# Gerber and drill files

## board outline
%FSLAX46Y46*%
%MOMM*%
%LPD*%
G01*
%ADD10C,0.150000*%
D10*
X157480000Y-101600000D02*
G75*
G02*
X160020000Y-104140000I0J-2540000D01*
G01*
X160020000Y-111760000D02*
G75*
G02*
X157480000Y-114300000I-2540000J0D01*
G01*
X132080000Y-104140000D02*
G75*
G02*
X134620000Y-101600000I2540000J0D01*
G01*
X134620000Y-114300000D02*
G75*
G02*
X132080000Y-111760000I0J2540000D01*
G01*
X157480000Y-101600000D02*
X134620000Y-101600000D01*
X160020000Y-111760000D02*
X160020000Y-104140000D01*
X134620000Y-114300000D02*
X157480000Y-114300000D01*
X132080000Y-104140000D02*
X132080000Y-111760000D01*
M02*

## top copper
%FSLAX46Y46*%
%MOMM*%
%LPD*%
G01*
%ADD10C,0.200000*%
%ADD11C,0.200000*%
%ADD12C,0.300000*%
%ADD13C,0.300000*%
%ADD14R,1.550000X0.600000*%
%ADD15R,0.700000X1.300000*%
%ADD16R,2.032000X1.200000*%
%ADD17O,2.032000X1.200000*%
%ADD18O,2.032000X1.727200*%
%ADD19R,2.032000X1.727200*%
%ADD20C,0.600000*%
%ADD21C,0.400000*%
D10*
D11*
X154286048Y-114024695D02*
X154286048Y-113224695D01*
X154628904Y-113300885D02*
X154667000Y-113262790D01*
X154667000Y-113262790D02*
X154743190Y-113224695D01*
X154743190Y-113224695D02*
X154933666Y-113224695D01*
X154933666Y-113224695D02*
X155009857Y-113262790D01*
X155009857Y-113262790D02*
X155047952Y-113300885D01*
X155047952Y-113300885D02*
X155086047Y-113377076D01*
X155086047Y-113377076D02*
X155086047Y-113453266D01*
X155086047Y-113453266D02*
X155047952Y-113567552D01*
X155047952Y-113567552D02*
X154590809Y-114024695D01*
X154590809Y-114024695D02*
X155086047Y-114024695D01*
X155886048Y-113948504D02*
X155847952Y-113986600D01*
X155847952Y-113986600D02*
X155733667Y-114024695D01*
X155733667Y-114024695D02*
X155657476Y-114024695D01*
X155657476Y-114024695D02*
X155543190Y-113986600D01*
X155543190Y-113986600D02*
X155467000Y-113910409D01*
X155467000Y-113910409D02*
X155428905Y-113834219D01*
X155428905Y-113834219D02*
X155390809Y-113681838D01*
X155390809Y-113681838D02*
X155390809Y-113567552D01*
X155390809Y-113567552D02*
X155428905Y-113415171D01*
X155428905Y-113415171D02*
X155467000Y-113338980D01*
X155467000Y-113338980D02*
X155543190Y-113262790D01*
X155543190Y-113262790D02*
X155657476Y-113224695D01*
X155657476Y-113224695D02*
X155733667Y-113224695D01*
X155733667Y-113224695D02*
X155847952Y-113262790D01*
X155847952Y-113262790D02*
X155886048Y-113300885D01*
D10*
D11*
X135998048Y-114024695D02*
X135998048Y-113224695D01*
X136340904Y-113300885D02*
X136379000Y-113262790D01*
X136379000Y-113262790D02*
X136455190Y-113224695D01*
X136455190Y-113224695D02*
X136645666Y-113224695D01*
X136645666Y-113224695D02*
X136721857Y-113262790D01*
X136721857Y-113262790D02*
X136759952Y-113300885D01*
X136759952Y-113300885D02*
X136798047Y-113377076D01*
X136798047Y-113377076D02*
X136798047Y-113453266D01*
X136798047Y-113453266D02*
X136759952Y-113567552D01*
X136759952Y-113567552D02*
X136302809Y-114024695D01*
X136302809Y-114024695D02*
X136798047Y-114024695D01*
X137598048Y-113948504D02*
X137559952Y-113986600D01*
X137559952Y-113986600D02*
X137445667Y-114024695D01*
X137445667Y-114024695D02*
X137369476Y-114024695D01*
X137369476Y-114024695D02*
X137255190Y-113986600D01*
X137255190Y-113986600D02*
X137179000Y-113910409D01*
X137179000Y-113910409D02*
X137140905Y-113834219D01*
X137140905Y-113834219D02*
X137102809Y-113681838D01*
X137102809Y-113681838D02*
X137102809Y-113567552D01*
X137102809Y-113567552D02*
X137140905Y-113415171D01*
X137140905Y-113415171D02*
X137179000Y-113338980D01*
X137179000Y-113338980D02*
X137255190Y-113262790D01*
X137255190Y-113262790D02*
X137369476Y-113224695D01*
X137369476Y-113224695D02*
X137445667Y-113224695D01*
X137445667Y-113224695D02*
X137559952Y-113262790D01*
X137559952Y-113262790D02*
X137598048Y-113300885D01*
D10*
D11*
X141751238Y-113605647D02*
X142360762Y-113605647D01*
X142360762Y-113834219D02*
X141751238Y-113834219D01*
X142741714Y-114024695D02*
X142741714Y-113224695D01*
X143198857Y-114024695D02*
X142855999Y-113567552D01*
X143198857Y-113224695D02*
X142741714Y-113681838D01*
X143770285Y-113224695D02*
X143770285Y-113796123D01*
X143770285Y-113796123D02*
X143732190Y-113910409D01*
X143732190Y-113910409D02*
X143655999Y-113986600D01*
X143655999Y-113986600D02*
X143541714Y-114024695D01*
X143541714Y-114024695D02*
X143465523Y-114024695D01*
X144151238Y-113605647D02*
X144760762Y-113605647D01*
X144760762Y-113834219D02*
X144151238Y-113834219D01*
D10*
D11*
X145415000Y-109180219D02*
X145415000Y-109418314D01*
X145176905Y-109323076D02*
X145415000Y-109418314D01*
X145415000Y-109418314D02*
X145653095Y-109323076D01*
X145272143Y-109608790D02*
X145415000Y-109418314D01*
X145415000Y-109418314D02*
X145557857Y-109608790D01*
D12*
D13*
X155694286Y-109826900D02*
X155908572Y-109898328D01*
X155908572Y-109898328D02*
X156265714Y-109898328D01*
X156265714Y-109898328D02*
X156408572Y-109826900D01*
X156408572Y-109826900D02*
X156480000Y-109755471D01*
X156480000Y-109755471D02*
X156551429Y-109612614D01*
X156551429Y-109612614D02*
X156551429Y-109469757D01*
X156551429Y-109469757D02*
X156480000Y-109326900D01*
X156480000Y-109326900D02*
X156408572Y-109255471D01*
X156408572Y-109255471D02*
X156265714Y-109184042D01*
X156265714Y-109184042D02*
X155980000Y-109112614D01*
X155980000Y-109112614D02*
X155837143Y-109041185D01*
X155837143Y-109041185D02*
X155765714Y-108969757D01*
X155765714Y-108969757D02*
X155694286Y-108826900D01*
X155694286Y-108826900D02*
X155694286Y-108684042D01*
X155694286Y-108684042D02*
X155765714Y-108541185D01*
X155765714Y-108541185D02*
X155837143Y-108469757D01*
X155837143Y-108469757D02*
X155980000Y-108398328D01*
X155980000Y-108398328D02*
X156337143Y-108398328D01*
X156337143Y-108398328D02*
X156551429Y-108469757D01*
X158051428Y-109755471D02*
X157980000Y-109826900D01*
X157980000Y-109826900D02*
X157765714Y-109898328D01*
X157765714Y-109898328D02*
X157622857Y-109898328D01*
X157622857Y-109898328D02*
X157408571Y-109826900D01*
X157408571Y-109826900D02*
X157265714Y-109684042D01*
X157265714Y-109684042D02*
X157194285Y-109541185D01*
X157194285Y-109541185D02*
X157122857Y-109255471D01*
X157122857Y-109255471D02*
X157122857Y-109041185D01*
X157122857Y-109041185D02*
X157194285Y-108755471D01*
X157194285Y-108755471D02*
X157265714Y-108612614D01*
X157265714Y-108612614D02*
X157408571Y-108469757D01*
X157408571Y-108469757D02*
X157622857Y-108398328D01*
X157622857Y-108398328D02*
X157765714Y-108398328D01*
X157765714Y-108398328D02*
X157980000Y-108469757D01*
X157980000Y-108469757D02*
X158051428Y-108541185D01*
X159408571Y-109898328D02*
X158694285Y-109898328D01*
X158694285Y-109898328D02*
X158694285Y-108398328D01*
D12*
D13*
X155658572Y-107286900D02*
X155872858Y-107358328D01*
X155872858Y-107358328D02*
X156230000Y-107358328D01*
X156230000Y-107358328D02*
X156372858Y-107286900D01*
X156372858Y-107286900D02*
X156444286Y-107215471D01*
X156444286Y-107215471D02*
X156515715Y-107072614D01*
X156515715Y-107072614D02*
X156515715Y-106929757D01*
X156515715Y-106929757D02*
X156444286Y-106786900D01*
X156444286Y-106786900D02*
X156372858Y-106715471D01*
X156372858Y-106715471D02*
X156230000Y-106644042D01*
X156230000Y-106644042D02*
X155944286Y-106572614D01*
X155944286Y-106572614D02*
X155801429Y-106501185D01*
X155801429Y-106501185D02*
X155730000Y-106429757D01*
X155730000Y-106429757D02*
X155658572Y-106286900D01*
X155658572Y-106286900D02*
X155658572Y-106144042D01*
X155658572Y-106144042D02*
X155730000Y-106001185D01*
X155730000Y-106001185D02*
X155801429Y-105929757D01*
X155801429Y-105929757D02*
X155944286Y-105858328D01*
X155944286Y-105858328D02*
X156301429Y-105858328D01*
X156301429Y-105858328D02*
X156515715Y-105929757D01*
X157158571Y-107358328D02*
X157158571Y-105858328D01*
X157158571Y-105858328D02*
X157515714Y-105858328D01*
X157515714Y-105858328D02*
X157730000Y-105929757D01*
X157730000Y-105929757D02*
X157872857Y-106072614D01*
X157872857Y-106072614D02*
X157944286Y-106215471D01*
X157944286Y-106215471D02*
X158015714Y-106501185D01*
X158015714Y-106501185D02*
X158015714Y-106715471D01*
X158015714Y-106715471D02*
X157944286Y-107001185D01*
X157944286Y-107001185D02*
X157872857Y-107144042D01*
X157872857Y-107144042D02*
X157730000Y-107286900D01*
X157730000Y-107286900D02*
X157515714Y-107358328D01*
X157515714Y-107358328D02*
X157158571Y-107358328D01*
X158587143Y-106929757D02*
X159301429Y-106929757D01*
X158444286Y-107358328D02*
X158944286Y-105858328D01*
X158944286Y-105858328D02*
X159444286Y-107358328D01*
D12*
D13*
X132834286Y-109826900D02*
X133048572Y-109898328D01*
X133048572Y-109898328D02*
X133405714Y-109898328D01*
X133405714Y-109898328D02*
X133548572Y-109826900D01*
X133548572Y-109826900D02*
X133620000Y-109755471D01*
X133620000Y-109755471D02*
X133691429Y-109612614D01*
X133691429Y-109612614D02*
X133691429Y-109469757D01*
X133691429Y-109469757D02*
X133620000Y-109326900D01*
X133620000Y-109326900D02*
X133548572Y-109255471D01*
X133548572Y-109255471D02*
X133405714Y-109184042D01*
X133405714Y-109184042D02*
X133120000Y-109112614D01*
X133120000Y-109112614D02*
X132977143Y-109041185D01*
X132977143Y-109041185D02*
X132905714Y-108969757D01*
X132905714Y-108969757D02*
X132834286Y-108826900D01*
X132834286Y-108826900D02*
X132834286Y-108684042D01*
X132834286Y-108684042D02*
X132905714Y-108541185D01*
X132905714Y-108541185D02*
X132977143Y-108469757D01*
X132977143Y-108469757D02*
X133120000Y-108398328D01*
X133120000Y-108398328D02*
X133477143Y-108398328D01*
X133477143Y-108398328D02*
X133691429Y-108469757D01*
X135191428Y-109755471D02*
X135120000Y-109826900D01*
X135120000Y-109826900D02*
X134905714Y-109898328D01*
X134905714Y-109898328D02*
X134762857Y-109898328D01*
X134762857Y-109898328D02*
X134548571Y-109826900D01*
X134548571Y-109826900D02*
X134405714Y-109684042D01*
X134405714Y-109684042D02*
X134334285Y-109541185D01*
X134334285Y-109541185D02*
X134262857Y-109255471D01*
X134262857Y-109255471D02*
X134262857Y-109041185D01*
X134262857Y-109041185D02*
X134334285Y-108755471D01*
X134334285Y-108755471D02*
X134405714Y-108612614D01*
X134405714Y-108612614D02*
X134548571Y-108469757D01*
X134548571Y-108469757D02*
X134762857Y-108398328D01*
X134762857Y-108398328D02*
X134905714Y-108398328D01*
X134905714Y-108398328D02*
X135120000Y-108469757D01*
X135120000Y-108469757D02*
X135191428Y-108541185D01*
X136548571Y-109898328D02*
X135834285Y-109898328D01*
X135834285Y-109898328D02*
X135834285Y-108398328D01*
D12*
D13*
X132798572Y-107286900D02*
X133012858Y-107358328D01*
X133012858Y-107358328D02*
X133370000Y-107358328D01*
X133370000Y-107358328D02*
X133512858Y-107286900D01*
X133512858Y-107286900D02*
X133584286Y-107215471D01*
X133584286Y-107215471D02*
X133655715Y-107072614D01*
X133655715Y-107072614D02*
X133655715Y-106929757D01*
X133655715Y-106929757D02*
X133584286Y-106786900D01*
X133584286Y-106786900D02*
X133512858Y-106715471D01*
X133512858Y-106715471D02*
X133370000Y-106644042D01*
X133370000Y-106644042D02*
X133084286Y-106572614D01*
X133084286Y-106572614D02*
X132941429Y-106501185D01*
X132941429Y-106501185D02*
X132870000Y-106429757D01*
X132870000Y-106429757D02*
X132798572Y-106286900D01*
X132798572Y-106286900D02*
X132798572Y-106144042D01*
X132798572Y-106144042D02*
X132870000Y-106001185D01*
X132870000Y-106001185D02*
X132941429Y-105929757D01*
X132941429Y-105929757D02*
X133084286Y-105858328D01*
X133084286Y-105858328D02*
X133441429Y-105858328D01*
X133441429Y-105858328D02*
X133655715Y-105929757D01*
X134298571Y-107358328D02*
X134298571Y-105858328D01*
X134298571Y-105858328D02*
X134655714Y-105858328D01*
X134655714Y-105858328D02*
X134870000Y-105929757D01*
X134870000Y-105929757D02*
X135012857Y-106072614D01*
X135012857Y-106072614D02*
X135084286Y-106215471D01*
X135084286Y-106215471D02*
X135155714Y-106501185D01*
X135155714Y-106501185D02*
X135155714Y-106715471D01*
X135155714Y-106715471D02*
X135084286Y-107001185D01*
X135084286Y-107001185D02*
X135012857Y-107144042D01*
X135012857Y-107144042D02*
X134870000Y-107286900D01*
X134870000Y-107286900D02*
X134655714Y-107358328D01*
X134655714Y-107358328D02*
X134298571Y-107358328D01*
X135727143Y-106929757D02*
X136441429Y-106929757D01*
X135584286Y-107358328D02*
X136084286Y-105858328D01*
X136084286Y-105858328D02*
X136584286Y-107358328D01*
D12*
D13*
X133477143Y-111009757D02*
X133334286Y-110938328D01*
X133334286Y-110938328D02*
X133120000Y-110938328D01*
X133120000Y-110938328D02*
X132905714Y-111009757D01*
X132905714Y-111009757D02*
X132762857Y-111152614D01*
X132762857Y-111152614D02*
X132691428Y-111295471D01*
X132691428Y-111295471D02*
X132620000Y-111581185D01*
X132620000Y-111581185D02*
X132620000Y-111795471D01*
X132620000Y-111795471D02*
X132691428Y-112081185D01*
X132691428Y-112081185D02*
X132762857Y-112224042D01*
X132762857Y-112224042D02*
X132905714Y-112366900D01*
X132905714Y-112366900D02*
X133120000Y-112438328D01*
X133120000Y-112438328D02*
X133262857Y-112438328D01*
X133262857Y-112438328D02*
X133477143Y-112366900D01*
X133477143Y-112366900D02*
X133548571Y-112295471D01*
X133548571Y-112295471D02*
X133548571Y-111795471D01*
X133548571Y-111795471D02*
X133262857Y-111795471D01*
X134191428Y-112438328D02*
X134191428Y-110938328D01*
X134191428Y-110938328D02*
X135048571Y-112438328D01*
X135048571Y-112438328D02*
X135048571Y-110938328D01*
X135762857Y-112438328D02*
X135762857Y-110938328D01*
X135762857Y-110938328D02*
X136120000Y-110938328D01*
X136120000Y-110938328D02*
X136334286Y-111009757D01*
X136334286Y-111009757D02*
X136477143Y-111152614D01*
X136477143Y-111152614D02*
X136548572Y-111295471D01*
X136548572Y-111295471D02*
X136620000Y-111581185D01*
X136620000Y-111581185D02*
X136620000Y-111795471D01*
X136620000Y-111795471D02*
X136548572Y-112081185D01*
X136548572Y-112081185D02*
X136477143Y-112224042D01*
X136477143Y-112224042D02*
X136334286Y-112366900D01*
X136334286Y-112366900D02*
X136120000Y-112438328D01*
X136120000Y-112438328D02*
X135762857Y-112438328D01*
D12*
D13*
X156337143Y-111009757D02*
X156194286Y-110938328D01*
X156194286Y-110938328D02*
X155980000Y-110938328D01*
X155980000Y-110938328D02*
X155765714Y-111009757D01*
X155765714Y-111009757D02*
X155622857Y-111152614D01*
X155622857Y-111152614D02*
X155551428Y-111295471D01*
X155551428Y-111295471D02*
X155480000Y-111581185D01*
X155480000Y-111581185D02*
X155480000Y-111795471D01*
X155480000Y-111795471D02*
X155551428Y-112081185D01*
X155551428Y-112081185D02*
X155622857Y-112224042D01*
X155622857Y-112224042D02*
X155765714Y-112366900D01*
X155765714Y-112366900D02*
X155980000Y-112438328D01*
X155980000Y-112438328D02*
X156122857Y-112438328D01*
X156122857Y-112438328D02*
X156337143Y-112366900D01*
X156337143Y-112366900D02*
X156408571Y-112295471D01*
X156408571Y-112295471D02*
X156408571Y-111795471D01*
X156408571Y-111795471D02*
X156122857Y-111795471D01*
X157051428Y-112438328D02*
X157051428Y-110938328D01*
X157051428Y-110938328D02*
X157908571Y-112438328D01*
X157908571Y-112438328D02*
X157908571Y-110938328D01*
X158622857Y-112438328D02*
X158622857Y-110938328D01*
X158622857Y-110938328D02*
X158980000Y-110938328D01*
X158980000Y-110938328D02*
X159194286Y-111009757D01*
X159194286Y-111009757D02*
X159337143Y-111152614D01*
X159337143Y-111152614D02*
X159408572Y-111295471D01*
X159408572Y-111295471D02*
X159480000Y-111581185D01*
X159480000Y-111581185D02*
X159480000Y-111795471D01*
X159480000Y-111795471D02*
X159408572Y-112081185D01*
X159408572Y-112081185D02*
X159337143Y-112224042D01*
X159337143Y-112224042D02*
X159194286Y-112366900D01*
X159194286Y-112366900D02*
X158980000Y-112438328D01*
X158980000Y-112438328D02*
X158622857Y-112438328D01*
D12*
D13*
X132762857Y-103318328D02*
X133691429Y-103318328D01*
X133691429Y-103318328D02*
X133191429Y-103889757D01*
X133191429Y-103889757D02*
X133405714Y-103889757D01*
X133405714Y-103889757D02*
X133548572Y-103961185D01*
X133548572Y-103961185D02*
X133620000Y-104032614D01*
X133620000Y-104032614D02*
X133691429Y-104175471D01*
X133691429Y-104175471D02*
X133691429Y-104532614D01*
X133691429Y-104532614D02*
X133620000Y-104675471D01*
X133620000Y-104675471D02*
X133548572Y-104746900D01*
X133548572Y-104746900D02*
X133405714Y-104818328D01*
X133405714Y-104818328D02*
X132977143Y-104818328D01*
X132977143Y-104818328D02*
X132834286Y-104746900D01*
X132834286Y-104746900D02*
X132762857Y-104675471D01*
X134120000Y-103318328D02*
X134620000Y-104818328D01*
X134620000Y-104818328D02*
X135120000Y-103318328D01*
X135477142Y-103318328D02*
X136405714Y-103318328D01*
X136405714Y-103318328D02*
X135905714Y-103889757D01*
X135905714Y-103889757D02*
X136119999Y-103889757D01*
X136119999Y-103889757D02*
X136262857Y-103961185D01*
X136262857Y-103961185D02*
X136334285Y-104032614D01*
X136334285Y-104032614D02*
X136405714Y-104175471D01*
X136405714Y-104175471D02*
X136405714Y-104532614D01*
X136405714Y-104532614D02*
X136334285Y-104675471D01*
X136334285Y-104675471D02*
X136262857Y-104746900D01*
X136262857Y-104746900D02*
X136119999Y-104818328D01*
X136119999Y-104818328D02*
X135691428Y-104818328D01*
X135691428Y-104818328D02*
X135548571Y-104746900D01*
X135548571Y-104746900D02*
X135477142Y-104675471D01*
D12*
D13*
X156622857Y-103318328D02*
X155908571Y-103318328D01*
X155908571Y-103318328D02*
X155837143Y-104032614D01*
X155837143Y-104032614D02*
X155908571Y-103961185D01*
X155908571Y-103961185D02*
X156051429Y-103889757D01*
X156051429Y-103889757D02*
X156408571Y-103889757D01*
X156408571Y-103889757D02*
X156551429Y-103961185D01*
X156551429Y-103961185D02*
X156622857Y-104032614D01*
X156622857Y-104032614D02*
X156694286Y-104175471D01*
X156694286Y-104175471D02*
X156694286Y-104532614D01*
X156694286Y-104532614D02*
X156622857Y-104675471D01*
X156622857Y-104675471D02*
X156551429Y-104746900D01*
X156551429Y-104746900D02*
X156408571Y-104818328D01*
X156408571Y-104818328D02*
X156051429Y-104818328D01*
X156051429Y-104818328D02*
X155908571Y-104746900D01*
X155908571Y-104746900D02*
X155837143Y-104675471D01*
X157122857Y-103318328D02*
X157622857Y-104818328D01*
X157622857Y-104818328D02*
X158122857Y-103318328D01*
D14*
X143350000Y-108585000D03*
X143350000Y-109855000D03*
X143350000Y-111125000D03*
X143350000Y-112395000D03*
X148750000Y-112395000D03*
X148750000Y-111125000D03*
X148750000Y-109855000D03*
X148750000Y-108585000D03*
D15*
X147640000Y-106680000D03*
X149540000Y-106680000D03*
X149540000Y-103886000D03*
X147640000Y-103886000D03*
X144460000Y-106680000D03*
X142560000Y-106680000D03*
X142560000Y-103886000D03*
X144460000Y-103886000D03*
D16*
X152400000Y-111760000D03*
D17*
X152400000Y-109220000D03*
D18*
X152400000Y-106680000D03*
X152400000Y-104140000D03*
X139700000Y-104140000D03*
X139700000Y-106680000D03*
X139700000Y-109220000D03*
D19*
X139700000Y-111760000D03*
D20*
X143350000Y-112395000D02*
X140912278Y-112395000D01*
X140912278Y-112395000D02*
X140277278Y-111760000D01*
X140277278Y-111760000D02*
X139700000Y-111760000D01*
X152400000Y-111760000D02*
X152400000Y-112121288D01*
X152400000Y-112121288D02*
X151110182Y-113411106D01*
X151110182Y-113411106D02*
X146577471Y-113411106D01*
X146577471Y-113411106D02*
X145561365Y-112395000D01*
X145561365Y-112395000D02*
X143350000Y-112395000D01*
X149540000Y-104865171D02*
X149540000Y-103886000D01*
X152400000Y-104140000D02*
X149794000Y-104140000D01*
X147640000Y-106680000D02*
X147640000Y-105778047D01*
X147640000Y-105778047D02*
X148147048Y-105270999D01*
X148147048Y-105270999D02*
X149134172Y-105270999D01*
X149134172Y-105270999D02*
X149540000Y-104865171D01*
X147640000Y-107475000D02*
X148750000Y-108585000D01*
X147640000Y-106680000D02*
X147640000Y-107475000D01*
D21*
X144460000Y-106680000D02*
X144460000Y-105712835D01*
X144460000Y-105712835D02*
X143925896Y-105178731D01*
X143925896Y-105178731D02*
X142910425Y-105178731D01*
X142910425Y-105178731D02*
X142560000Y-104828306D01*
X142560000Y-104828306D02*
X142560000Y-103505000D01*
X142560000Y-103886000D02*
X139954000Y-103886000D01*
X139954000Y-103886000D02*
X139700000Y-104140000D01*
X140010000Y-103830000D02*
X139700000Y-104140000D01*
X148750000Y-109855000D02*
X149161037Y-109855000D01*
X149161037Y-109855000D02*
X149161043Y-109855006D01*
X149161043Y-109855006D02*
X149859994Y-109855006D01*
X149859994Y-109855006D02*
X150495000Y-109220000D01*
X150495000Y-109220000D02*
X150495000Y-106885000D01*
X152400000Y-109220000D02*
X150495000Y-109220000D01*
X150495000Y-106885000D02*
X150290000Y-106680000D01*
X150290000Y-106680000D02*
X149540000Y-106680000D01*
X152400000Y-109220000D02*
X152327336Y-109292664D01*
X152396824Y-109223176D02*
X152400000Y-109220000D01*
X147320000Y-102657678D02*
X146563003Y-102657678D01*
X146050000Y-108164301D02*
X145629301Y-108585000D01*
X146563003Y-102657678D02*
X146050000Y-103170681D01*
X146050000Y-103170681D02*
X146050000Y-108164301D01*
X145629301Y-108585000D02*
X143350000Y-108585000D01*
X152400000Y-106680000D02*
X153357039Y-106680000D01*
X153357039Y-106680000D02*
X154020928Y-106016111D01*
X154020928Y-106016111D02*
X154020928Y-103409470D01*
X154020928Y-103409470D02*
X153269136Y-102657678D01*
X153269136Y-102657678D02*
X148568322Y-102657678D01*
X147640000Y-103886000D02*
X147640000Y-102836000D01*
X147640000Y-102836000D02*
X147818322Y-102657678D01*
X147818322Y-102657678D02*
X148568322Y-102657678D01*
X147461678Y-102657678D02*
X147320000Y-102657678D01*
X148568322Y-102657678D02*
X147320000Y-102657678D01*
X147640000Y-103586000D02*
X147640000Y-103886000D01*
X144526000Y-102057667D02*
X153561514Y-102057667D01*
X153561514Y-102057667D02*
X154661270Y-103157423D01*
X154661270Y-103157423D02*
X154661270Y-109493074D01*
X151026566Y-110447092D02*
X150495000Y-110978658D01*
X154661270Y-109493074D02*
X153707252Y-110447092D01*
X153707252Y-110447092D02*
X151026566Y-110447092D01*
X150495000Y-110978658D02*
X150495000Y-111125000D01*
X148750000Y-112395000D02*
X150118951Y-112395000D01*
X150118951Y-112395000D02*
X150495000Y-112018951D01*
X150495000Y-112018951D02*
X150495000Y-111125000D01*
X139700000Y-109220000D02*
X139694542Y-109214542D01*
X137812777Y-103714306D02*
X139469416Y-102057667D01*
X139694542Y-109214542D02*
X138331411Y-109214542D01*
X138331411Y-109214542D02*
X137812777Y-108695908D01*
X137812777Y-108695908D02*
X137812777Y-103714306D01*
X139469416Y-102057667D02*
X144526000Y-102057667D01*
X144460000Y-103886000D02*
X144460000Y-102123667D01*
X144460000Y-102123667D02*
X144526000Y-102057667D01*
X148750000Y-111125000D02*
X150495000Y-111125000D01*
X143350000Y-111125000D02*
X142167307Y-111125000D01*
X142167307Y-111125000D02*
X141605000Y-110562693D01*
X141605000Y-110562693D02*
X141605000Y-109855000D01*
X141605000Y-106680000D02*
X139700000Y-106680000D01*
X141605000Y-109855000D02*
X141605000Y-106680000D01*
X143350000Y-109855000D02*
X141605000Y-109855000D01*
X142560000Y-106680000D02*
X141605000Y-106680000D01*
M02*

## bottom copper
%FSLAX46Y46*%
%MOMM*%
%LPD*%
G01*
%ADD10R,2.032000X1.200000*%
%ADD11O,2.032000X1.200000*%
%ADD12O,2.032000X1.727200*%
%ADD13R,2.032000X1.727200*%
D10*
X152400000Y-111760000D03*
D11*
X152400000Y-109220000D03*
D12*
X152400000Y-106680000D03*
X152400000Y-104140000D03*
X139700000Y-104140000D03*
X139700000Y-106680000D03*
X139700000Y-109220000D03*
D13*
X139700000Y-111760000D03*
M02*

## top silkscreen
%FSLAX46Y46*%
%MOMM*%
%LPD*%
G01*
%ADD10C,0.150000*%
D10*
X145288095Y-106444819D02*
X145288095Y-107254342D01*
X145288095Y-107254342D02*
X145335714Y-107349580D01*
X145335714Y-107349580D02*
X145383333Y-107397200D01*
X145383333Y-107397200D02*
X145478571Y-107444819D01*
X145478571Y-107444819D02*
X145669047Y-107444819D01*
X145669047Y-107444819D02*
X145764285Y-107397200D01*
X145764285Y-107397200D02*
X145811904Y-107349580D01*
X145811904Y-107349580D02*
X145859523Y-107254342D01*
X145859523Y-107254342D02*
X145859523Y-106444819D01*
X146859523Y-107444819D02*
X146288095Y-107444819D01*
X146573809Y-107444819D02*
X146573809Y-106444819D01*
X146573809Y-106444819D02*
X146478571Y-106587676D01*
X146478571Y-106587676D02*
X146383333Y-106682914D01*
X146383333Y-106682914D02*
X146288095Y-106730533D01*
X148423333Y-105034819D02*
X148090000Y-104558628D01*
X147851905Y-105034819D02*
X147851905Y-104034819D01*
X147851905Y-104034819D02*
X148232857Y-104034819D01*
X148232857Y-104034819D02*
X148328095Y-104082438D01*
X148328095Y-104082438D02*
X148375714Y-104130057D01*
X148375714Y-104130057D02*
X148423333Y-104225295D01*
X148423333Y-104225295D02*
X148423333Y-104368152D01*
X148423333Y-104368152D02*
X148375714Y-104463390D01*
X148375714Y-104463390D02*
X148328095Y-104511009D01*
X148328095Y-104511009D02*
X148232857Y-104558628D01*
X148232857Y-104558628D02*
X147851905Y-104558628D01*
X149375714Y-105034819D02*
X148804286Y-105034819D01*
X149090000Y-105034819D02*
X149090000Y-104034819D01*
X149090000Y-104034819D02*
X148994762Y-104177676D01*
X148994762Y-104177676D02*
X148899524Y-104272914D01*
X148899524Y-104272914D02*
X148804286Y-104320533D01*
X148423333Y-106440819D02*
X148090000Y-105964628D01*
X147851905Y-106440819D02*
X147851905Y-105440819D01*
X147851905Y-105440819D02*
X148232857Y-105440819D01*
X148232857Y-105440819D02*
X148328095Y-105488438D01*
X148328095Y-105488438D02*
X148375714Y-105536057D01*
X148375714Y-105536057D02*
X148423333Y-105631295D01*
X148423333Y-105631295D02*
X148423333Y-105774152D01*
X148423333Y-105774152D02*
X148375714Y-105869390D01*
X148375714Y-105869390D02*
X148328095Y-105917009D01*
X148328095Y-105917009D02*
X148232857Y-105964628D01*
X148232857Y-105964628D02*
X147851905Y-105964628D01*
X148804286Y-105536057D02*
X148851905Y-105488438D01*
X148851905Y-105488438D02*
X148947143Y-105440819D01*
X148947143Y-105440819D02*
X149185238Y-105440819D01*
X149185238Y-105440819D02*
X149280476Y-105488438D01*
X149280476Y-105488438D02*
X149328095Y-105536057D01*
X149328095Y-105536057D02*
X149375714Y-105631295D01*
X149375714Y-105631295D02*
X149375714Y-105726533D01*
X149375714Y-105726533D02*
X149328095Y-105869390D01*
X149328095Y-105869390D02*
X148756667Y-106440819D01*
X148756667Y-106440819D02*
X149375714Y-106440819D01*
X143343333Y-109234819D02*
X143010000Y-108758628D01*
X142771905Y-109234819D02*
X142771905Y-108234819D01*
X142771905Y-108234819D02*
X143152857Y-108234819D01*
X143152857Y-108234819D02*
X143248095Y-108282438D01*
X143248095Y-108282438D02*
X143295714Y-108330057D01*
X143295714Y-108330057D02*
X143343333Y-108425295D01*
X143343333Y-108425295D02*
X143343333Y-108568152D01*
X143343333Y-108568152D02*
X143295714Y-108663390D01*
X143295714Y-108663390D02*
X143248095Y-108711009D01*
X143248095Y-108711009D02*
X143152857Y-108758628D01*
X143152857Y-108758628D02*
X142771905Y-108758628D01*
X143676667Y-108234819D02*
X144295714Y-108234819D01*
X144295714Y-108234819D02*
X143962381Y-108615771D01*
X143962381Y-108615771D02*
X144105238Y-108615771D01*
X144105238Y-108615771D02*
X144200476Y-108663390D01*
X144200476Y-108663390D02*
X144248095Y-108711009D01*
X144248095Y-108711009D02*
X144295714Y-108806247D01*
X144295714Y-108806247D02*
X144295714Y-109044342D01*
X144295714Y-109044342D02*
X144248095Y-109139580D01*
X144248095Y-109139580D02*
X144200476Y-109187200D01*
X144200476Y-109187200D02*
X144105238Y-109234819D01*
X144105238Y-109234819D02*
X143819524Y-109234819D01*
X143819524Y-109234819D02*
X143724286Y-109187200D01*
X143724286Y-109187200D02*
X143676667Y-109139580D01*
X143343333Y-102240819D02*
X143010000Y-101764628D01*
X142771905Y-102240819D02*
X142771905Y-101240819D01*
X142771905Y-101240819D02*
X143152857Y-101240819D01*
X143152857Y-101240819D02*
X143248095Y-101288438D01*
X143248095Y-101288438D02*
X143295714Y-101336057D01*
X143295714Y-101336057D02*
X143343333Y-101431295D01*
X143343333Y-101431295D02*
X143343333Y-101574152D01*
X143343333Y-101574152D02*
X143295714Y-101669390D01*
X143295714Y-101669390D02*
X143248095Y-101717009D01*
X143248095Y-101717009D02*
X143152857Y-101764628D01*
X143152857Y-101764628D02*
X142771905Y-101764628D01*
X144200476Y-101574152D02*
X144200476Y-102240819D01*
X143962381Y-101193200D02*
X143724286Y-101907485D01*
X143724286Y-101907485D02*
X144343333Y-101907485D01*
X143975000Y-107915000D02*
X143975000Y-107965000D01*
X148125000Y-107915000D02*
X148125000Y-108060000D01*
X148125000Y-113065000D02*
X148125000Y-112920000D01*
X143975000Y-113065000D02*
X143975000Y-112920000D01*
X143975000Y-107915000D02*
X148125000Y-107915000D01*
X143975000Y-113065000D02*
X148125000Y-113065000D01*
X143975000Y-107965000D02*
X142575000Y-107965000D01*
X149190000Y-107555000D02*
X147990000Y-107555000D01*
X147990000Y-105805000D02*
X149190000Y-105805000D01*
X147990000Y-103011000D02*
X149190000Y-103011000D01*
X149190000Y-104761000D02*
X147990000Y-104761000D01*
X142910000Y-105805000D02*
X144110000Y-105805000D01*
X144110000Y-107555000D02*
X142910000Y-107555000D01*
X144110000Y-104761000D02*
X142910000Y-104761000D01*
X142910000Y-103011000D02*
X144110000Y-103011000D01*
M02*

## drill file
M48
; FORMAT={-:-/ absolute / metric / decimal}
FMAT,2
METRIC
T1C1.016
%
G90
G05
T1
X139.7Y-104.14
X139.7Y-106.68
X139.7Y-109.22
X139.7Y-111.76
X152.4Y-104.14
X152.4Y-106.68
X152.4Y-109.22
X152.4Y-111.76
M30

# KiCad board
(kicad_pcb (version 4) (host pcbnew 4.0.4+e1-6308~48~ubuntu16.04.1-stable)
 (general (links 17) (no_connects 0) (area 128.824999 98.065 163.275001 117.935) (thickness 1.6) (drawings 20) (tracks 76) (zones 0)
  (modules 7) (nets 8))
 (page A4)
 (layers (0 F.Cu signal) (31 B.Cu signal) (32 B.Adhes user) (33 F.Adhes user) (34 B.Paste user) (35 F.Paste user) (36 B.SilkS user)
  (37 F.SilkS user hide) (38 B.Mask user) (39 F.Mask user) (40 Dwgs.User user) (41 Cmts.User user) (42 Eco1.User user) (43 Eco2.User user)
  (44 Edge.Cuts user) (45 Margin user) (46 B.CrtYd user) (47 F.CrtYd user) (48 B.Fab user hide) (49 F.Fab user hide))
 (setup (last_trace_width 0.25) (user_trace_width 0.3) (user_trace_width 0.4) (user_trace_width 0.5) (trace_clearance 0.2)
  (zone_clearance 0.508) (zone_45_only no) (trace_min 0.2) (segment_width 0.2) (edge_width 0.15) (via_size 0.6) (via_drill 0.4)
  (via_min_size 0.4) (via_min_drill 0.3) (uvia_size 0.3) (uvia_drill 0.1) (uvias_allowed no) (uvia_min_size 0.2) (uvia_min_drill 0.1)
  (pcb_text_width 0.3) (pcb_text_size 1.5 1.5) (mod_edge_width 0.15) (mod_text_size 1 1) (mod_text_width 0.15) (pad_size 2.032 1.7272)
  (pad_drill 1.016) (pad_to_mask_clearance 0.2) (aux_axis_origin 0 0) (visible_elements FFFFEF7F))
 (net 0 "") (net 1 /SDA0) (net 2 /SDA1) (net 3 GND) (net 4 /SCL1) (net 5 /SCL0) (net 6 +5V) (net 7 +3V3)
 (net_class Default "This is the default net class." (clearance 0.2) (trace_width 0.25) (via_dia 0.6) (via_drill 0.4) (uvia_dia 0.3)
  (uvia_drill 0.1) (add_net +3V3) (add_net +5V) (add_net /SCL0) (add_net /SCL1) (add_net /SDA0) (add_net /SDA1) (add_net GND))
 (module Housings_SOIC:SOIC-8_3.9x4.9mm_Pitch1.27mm (layer F.Cu) (at 146.05 110.49)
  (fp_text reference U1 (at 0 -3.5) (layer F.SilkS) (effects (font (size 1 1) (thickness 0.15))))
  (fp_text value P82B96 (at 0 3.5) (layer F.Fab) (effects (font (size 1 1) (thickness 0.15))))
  (fp_line (start -2.075 -2.575) (end -2.075 -2.525) (layer F.SilkS) (width 0.15))
  (fp_line (start 2.075 -2.575) (end 2.075 -2.43) (layer F.SilkS) (width 0.15))
  (fp_line (start 2.075 2.575) (end 2.075 2.43) (layer F.SilkS) (width 0.15))
  (fp_line (start -2.075 2.575) (end -2.075 2.43) (layer F.SilkS) (width 0.15))
  (fp_line (start -2.075 -2.575) (end 2.075 -2.575) (layer F.SilkS) (width 0.15))
  (fp_line (start -2.075 2.575) (end 2.075 2.575) (layer F.SilkS) (width 0.15))
  (fp_line (start -2.075 -2.525) (end -3.475 -2.525) (layer F.SilkS) (width 0.15))
  (pad 1 smd rect (at -2.7 -1.905) (size 1.55 0.6) (layers F.Cu F.Paste F.Mask) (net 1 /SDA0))
  (pad 2 smd rect (at -2.7 -0.635) (size 1.55 0.6) (layers F.Cu F.Paste F.Mask) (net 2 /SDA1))
  (pad 3 smd rect (at -2.7 0.635) (size 1.55 0.6) (layers F.Cu F.Paste F.Mask) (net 2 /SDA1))
  (pad 4 smd rect (at -2.7 1.905) (size 1.55 0.6) (layers F.Cu F.Paste F.Mask) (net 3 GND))
  (pad 5 smd rect (at 2.7 1.905) (size 1.55 0.6) (layers F.Cu F.Paste F.Mask) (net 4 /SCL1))
  (pad 6 smd rect (at 2.7 0.635) (size 1.55 0.6) (layers F.Cu F.Paste F.Mask) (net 4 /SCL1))
  (pad 7 smd rect (at 2.7 -0.635) (size 1.55 0.6) (layers F.Cu F.Paste F.Mask) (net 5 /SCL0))
  (pad 8 smd rect (at 2.7 -1.905) (size 1.55 0.6) (layers F.Cu F.Paste F.Mask) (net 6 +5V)))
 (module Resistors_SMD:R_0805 (layer F.Cu) (at 148.59 106.68)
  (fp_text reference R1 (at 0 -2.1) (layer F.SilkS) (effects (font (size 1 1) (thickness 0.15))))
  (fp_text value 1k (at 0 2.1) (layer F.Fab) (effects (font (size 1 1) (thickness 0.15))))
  (fp_line (start 0.6 0.875) (end -0.6 0.875) (layer F.SilkS) (width 0.15))
  (fp_line (start -0.6 -0.875) (end 0.6 -0.875) (layer F.SilkS) (width 0.15))
  (pad 1 smd rect (at -0.95 0) (size 0.7 1.3) (layers F.Cu F.Paste F.Mask) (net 6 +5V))
  (pad 2 smd rect (at 0.95 0) (size 0.7 1.3) (layers F.Cu F.Paste F.Mask) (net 5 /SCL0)))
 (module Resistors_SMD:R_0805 (layer F.Cu) (at 148.59 103.886 180)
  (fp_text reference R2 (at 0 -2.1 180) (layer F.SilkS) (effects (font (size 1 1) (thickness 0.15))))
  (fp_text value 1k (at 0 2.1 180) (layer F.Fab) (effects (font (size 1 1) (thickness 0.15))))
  (fp_line (start 0.6 0.875) (end -0.6 0.875) (layer F.SilkS) (width 0.15))
  (fp_line (start -0.6 -0.875) (end 0.6 -0.875) (layer F.SilkS) (width 0.15))
  (pad 1 smd rect (at -0.95 0 180) (size 0.7 1.3) (layers F.Cu F.Paste F.Mask) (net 6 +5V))
  (pad 2 smd rect (at 0.95 0 180) (size 0.7 1.3) (layers F.Cu F.Paste F.Mask) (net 1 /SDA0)))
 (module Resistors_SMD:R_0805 (layer F.Cu) (at 143.51 106.68 180)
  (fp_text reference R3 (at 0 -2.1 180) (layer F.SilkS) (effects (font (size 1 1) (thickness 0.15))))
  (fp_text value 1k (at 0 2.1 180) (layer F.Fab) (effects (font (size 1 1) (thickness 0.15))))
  (fp_line (start 0.6 0.875) (end -0.6 0.875) (layer F.SilkS) (width 0.15))
  (fp_line (start -0.6 -0.875) (end 0.6 -0.875) (layer F.SilkS) (width 0.15))
  (pad 1 smd rect (at -0.95 0 180) (size 0.7 1.3) (layers F.Cu F.Paste F.Mask) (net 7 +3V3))
  (pad 2 smd rect (at 0.95 0 180) (size 0.7 1.3) (layers F.Cu F.Paste F.Mask) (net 2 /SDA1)))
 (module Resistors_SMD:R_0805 (layer F.Cu) (at 143.51 103.886)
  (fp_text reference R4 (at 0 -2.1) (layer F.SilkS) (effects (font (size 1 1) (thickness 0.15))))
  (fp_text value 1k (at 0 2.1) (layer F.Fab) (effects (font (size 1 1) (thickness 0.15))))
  (fp_line (start 0.6 0.875) (end -0.6 0.875) (layer F.SilkS) (width 0.15))
  (fp_line (start -0.6 -0.875) (end 0.6 -0.875) (layer F.SilkS) (width 0.15))
  (pad 1 smd rect (at -0.95 0) (size 0.7 1.3) (layers F.Cu F.Paste F.Mask) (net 7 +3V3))
  (pad 2 smd rect (at 0.95 0) (size 0.7 1.3) (layers F.Cu F.Paste F.Mask) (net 4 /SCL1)))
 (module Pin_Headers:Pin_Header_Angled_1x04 (layer B.Cu) (at 152.4 111.76)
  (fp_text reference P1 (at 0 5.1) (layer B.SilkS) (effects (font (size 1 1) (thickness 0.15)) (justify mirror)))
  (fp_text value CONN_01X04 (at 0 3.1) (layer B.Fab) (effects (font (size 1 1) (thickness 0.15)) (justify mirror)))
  (pad 1 thru_hole rect (at 0 0) (size 2.032 1.2) (drill 1.016) (layers *.Cu *.Mask) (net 3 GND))
  (pad 2 thru_hole oval (at 0 -2.54) (size 2.032 1.2) (drill 1.016) (layers *.Cu *.Mask) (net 5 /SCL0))
  (pad 3 thru_hole oval (at 0 -5.08) (size 2.032 1.7272) (drill 1.016) (layers *.Cu *.Mask) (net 1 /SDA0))
  (pad 4 thru_hole oval (at 0 -7.62) (size 2.032 1.7272) (drill 1.016) (layers *.Cu *.Mask) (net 6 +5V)))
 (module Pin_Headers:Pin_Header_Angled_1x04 (layer B.Cu) (at 139.7 104.14 180)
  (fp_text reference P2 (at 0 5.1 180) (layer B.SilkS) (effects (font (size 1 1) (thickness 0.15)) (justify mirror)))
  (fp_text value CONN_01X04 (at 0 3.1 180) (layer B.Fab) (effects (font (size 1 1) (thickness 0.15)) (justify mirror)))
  (pad 1 thru_hole oval (at 0 0 180) (size 2.032 1.7272) (drill 1.016) (layers *.Cu *.Mask) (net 7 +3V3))
  (pad 2 thru_hole oval (at 0 -2.54 180) (size 2.032 1.7272) (drill 1.016) (layers *.Cu *.Mask) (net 2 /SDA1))
  (pad 3 thru_hole oval (at 0 -5.08 180) (size 2.032 1.7272) (drill 1.016) (layers *.Cu *.Mask) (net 4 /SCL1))
  (pad 4 thru_hole rect (at 0 -7.62 180) (size 2.032 1.7272) (drill 1.016) (layers *.Cu *.Mask) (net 3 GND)))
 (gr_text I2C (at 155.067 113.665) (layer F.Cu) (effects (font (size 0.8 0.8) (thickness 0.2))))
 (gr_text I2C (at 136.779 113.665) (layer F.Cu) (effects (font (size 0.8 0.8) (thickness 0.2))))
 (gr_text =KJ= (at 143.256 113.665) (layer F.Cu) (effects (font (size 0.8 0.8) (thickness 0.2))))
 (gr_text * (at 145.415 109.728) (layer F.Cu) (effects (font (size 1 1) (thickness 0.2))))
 (gr_arc (start 157.48 104.14) (end 157.48 101.6) (angle 90) (layer Edge.Cuts) (width 0.15))
 (gr_arc (start 157.48 111.76) (end 160.02 111.76) (angle 90) (layer Edge.Cuts) (width 0.15))
 (gr_arc (start 134.62 104.14) (end 132.08 104.14) (angle 90) (layer Edge.Cuts) (width 0.15))
 (gr_arc (start 134.62 111.76) (end 134.62 114.3) (angle 90) (layer Edge.Cuts) (width 0.15))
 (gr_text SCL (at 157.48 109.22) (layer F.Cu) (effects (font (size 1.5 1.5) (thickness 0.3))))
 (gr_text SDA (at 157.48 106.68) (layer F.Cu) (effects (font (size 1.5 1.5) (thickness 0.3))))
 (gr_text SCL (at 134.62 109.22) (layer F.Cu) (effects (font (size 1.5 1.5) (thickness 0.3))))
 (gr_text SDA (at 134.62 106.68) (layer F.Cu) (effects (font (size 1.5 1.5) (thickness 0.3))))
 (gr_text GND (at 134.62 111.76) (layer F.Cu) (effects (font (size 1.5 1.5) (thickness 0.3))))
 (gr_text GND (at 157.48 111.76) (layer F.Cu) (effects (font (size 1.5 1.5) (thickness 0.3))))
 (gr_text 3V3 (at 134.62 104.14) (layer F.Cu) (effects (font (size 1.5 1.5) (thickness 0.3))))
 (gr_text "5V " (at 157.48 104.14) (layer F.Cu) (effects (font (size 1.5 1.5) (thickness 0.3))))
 (gr_line (start 157.48 101.6) (end 134.62 101.6) (layer Edge.Cuts) (width 0.15))
 (gr_line (start 160.02 111.76) (end 160.02 104.14) (layer Edge.Cuts) (width 0.15))
 (gr_line (start 134.62 114.3) (end 157.48 114.3) (layer Edge.Cuts) (width 0.15))
 (gr_line (start 132.08 104.14) (end 132.08 111.76) (layer Edge.Cuts) (width 0.15))
 (segment (start 143.35 112.395) (end 140.912278 112.395) (width 0.6) (layer F.Cu) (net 3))
 (segment (start 140.912278 112.395) (end 140.277278 111.76) (width 0.6) (layer F.Cu) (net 3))
 (segment (start 140.277278 111.76) (end 139.7 111.76) (width 0.6) (layer F.Cu) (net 3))
 (segment (start 152.4 111.76) (end 152.4 112.121288) (width 0.6) (layer F.Cu) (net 3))
 (segment (start 152.4 112.121288) (end 151.110182 113.411106) (width 0.6) (layer F.Cu) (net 3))
 (segment (start 151.110182 113.411106) (end 146.577471 113.411106) (width 0.6) (layer F.Cu) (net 3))
 (segment (start 146.577471 113.411106) (end 145.561365 112.395) (width 0.6) (layer F.Cu) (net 3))
 (segment (start 145.561365 112.395) (end 143.35 112.395) (width 0.6) (layer F.Cu) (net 3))
 (segment (start 149.54 104.865171) (end 149.54 103.886) (width 0.6) (layer F.Cu) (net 6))
 (segment (start 152.4 104.14) (end 149.794 104.14) (width 0.6) (layer F.Cu) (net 6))
 (segment (start 147.64 106.68) (end 147.64 105.778047) (width 0.6) (layer F.Cu) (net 6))
 (segment (start 147.64 105.778047) (end 148.147048 105.270999) (width 0.6) (layer F.Cu) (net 6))
 (segment (start 148.147048 105.270999) (end 149.134172 105.270999) (width 0.6) (layer F.Cu) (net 6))
 (segment (start 149.134172 105.270999) (end 149.54 104.865171) (width 0.6) (layer F.Cu) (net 6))
 (segment (start 147.64 107.475) (end 148.75 108.585) (width 0.6) (layer F.Cu) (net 6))
 (segment (start 147.64 106.68) (end 147.64 107.475) (width 0.6) (layer F.Cu) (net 6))
 (segment (start 144.46 106.68) (end 144.46 105.712835) (width 0.4) (layer F.Cu) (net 7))
 (segment (start 144.46 105.712835) (end 143.925896 105.178731) (width 0.4) (layer F.Cu) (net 7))
 (segment (start 143.925896 105.178731) (end 142.910425 105.178731) (width 0.4) (layer F.Cu) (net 7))
 (segment (start 142.910425 105.178731) (end 142.56 104.828306) (width 0.4) (layer F.Cu) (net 7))
 (segment (start 142.56 104.828306) (end 142.56 103.505) (width 0.4) (layer F.Cu) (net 7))
 (segment (start 142.56 103.886) (end 139.954 103.886) (width 0.4) (layer F.Cu) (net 7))
 (segment (start 139.954 103.886) (end 139.7 104.14) (width 0.4) (layer F.Cu) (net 7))
 (segment (start 140.01 103.83) (end 139.7 104.14) (width 0.4) (layer F.Cu) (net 7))
 (segment (start 148.75 109.855) (end 149.161037 109.855) (width 0.4) (layer F.Cu) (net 5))
 (segment (start 149.161037 109.855) (end 149.161043 109.855006) (width 0.4) (layer F.Cu) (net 5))
 (segment (start 149.161043 109.855006) (end 149.859994 109.855006) (width 0.4) (layer F.Cu) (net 5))
 (segment (start 149.859994 109.855006) (end 150.495 109.22) (width 0.4) (layer F.Cu) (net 5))
 (segment (start 150.495 109.22) (end 150.495 106.885) (width 0.4) (layer F.Cu) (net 5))
 (segment (start 152.4 109.22) (end 150.495 109.22) (width 0.4) (layer F.Cu) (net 5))
 (segment (start 150.495 106.885) (end 150.29 106.68) (width 0.4) (layer F.Cu) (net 5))
 (segment (start 150.29 106.68) (end 149.54 106.68) (width 0.4) (layer F.Cu) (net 5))
 (segment (start 152.4 109.22) (end 152.327336 109.292664) (width 0.4) (layer F.Cu) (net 5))
 (segment (start 152.396824 109.223176) (end 152.4 109.22) (width 0.4) (layer F.Cu) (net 5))
 (segment (start 147.32 102.657678) (end 146.563003 102.657678) (width 0.4) (layer F.Cu) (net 1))
 (segment (start 146.05 108.164301) (end 145.629301 108.585) (width 0.4) (layer F.Cu) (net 1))
 (segment (start 146.563003 102.657678) (end 146.05 103.170681) (width 0.4) (layer F.Cu) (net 1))
 (segment (start 146.05 103.170681) (end 146.05 108.164301) (width 0.4) (layer F.Cu) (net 1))
 (segment (start 145.629301 108.585) (end 143.35 108.585) (width 0.4) (layer F.Cu) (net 1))
 (segment (start 152.4 106.68) (end 153.357039 106.68) (width 0.4) (layer F.Cu) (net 1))
 (segment (start 153.357039 106.68) (end 154.020928 106.016111) (width 0.4) (layer F.Cu) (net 1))
 (segment (start 154.020928 106.016111) (end 154.020928 103.40947) (width 0.4) (layer F.Cu) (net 1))
 (segment (start 154.020928 103.40947) (end 153.269136 102.657678) (width 0.4) (layer F.Cu) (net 1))
 (segment (start 153.269136 102.657678) (end 148.568322 102.657678) (width 0.4) (layer F.Cu) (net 1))
 (segment (start 147.64 103.886) (end 147.64 102.836) (width 0.4) (layer F.Cu) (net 1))
 (segment (start 147.64 102.836) (end 147.818322 102.657678) (width 0.4) (layer F.Cu) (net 1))
 (segment (start 147.818322 102.657678) (end 148.568322 102.657678) (width 0.4) (layer F.Cu) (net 1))
 (segment (start 147.461678 102.657678) (end 147.32 102.657678) (width 0.4) (layer F.Cu) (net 1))
 (segment (start 148.568322 102.657678) (end 147.32 102.657678) (width 0.4) (layer F.Cu) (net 1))
 (segment (start 147.64 103.586) (end 147.64 103.886) (width 0.4) (layer F.Cu) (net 1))
 (segment (start 144.526 102.057667) (end 153.561514 102.057667) (width 0.4) (layer F.Cu) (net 4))
 (segment (start 153.561514 102.057667) (end 154.66127 103.157423) (width 0.4) (layer F.Cu) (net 4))
 (segment (start 154.66127 103.157423) (end 154.66127 109.493074) (width 0.4) (layer F.Cu) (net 4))
 (segment (start 151.026566 110.447092) (end 150.495 110.978658) (width 0.4) (layer F.Cu) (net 4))
 (segment (start 154.66127 109.493074) (end 153.707252 110.447092) (width 0.4) (layer F.Cu) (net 4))
 (segment (start 153.707252 110.447092) (end 151.026566 110.447092) (width 0.4) (layer F.Cu) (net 4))
 (segment (start 150.495 110.978658) (end 150.495 111.125) (width 0.4) (layer F.Cu) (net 4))
 (segment (start 148.75 112.395) (end 150.118951 112.395) (width 0.4) (layer F.Cu) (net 4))
 (segment (start 150.118951 112.395) (end 150.495 112.018951) (width 0.4) (layer F.Cu) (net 4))
 (segment (start 150.495 112.018951) (end 150.495 111.125) (width 0.4) (layer F.Cu) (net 4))
 (segment (start 139.7 109.22) (end 139.694542 109.214542) (width 0.4) (layer F.Cu) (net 4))
 (segment (start 137.812777 103.714306) (end 139.469416 102.057667) (width 0.4) (layer F.Cu) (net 4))
 (segment (start 139.694542 109.214542) (end 138.331411 109.214542) (width 0.4) (layer F.Cu) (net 4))
 (segment (start 138.331411 109.214542) (end 137.812777 108.695908) (width 0.4) (layer F.Cu) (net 4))
 (segment (start 137.812777 108.695908) (end 137.812777 103.714306) (width 0.4) (layer F.Cu) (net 4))
 (segment (start 139.469416 102.057667) (end 144.526 102.057667) (width 0.4) (layer F.Cu) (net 4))
 (segment (start 144.46 103.886) (end 144.46 102.123667) (width 0.4) (layer F.Cu) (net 4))
 (segment (start 144.46 102.123667) (end 144.526 102.057667) (width 0.4) (layer F.Cu) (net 4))
 (segment (start 148.75 111.125) (end 150.495 111.125) (width 0.4) (layer F.Cu) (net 4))
 (segment (start 143.35 111.125) (end 142.167307 111.125) (width 0.4) (layer F.Cu) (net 2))
 (segment (start 142.167307 111.125) (end 141.605 110.562693) (width 0.4) (layer F.Cu) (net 2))
 (segment (start 141.605 110.562693) (end 141.605 109.855) (width 0.4) (layer F.Cu) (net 2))
 (segment (start 141.605 106.68) (end 139.7 106.68) (width 0.4) (layer F.Cu) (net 2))
 (segment (start 141.605 109.855) (end 141.605 106.68) (width 0.4) (layer F.Cu) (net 2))
 (segment (start 143.35 109.855) (end 141.605 109.855) (width 0.4) (layer F.Cu) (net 2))
 (segment (start 142.56 106.68) (end 141.605 106.68) (width 0.4) (layer F.Cu) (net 2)))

